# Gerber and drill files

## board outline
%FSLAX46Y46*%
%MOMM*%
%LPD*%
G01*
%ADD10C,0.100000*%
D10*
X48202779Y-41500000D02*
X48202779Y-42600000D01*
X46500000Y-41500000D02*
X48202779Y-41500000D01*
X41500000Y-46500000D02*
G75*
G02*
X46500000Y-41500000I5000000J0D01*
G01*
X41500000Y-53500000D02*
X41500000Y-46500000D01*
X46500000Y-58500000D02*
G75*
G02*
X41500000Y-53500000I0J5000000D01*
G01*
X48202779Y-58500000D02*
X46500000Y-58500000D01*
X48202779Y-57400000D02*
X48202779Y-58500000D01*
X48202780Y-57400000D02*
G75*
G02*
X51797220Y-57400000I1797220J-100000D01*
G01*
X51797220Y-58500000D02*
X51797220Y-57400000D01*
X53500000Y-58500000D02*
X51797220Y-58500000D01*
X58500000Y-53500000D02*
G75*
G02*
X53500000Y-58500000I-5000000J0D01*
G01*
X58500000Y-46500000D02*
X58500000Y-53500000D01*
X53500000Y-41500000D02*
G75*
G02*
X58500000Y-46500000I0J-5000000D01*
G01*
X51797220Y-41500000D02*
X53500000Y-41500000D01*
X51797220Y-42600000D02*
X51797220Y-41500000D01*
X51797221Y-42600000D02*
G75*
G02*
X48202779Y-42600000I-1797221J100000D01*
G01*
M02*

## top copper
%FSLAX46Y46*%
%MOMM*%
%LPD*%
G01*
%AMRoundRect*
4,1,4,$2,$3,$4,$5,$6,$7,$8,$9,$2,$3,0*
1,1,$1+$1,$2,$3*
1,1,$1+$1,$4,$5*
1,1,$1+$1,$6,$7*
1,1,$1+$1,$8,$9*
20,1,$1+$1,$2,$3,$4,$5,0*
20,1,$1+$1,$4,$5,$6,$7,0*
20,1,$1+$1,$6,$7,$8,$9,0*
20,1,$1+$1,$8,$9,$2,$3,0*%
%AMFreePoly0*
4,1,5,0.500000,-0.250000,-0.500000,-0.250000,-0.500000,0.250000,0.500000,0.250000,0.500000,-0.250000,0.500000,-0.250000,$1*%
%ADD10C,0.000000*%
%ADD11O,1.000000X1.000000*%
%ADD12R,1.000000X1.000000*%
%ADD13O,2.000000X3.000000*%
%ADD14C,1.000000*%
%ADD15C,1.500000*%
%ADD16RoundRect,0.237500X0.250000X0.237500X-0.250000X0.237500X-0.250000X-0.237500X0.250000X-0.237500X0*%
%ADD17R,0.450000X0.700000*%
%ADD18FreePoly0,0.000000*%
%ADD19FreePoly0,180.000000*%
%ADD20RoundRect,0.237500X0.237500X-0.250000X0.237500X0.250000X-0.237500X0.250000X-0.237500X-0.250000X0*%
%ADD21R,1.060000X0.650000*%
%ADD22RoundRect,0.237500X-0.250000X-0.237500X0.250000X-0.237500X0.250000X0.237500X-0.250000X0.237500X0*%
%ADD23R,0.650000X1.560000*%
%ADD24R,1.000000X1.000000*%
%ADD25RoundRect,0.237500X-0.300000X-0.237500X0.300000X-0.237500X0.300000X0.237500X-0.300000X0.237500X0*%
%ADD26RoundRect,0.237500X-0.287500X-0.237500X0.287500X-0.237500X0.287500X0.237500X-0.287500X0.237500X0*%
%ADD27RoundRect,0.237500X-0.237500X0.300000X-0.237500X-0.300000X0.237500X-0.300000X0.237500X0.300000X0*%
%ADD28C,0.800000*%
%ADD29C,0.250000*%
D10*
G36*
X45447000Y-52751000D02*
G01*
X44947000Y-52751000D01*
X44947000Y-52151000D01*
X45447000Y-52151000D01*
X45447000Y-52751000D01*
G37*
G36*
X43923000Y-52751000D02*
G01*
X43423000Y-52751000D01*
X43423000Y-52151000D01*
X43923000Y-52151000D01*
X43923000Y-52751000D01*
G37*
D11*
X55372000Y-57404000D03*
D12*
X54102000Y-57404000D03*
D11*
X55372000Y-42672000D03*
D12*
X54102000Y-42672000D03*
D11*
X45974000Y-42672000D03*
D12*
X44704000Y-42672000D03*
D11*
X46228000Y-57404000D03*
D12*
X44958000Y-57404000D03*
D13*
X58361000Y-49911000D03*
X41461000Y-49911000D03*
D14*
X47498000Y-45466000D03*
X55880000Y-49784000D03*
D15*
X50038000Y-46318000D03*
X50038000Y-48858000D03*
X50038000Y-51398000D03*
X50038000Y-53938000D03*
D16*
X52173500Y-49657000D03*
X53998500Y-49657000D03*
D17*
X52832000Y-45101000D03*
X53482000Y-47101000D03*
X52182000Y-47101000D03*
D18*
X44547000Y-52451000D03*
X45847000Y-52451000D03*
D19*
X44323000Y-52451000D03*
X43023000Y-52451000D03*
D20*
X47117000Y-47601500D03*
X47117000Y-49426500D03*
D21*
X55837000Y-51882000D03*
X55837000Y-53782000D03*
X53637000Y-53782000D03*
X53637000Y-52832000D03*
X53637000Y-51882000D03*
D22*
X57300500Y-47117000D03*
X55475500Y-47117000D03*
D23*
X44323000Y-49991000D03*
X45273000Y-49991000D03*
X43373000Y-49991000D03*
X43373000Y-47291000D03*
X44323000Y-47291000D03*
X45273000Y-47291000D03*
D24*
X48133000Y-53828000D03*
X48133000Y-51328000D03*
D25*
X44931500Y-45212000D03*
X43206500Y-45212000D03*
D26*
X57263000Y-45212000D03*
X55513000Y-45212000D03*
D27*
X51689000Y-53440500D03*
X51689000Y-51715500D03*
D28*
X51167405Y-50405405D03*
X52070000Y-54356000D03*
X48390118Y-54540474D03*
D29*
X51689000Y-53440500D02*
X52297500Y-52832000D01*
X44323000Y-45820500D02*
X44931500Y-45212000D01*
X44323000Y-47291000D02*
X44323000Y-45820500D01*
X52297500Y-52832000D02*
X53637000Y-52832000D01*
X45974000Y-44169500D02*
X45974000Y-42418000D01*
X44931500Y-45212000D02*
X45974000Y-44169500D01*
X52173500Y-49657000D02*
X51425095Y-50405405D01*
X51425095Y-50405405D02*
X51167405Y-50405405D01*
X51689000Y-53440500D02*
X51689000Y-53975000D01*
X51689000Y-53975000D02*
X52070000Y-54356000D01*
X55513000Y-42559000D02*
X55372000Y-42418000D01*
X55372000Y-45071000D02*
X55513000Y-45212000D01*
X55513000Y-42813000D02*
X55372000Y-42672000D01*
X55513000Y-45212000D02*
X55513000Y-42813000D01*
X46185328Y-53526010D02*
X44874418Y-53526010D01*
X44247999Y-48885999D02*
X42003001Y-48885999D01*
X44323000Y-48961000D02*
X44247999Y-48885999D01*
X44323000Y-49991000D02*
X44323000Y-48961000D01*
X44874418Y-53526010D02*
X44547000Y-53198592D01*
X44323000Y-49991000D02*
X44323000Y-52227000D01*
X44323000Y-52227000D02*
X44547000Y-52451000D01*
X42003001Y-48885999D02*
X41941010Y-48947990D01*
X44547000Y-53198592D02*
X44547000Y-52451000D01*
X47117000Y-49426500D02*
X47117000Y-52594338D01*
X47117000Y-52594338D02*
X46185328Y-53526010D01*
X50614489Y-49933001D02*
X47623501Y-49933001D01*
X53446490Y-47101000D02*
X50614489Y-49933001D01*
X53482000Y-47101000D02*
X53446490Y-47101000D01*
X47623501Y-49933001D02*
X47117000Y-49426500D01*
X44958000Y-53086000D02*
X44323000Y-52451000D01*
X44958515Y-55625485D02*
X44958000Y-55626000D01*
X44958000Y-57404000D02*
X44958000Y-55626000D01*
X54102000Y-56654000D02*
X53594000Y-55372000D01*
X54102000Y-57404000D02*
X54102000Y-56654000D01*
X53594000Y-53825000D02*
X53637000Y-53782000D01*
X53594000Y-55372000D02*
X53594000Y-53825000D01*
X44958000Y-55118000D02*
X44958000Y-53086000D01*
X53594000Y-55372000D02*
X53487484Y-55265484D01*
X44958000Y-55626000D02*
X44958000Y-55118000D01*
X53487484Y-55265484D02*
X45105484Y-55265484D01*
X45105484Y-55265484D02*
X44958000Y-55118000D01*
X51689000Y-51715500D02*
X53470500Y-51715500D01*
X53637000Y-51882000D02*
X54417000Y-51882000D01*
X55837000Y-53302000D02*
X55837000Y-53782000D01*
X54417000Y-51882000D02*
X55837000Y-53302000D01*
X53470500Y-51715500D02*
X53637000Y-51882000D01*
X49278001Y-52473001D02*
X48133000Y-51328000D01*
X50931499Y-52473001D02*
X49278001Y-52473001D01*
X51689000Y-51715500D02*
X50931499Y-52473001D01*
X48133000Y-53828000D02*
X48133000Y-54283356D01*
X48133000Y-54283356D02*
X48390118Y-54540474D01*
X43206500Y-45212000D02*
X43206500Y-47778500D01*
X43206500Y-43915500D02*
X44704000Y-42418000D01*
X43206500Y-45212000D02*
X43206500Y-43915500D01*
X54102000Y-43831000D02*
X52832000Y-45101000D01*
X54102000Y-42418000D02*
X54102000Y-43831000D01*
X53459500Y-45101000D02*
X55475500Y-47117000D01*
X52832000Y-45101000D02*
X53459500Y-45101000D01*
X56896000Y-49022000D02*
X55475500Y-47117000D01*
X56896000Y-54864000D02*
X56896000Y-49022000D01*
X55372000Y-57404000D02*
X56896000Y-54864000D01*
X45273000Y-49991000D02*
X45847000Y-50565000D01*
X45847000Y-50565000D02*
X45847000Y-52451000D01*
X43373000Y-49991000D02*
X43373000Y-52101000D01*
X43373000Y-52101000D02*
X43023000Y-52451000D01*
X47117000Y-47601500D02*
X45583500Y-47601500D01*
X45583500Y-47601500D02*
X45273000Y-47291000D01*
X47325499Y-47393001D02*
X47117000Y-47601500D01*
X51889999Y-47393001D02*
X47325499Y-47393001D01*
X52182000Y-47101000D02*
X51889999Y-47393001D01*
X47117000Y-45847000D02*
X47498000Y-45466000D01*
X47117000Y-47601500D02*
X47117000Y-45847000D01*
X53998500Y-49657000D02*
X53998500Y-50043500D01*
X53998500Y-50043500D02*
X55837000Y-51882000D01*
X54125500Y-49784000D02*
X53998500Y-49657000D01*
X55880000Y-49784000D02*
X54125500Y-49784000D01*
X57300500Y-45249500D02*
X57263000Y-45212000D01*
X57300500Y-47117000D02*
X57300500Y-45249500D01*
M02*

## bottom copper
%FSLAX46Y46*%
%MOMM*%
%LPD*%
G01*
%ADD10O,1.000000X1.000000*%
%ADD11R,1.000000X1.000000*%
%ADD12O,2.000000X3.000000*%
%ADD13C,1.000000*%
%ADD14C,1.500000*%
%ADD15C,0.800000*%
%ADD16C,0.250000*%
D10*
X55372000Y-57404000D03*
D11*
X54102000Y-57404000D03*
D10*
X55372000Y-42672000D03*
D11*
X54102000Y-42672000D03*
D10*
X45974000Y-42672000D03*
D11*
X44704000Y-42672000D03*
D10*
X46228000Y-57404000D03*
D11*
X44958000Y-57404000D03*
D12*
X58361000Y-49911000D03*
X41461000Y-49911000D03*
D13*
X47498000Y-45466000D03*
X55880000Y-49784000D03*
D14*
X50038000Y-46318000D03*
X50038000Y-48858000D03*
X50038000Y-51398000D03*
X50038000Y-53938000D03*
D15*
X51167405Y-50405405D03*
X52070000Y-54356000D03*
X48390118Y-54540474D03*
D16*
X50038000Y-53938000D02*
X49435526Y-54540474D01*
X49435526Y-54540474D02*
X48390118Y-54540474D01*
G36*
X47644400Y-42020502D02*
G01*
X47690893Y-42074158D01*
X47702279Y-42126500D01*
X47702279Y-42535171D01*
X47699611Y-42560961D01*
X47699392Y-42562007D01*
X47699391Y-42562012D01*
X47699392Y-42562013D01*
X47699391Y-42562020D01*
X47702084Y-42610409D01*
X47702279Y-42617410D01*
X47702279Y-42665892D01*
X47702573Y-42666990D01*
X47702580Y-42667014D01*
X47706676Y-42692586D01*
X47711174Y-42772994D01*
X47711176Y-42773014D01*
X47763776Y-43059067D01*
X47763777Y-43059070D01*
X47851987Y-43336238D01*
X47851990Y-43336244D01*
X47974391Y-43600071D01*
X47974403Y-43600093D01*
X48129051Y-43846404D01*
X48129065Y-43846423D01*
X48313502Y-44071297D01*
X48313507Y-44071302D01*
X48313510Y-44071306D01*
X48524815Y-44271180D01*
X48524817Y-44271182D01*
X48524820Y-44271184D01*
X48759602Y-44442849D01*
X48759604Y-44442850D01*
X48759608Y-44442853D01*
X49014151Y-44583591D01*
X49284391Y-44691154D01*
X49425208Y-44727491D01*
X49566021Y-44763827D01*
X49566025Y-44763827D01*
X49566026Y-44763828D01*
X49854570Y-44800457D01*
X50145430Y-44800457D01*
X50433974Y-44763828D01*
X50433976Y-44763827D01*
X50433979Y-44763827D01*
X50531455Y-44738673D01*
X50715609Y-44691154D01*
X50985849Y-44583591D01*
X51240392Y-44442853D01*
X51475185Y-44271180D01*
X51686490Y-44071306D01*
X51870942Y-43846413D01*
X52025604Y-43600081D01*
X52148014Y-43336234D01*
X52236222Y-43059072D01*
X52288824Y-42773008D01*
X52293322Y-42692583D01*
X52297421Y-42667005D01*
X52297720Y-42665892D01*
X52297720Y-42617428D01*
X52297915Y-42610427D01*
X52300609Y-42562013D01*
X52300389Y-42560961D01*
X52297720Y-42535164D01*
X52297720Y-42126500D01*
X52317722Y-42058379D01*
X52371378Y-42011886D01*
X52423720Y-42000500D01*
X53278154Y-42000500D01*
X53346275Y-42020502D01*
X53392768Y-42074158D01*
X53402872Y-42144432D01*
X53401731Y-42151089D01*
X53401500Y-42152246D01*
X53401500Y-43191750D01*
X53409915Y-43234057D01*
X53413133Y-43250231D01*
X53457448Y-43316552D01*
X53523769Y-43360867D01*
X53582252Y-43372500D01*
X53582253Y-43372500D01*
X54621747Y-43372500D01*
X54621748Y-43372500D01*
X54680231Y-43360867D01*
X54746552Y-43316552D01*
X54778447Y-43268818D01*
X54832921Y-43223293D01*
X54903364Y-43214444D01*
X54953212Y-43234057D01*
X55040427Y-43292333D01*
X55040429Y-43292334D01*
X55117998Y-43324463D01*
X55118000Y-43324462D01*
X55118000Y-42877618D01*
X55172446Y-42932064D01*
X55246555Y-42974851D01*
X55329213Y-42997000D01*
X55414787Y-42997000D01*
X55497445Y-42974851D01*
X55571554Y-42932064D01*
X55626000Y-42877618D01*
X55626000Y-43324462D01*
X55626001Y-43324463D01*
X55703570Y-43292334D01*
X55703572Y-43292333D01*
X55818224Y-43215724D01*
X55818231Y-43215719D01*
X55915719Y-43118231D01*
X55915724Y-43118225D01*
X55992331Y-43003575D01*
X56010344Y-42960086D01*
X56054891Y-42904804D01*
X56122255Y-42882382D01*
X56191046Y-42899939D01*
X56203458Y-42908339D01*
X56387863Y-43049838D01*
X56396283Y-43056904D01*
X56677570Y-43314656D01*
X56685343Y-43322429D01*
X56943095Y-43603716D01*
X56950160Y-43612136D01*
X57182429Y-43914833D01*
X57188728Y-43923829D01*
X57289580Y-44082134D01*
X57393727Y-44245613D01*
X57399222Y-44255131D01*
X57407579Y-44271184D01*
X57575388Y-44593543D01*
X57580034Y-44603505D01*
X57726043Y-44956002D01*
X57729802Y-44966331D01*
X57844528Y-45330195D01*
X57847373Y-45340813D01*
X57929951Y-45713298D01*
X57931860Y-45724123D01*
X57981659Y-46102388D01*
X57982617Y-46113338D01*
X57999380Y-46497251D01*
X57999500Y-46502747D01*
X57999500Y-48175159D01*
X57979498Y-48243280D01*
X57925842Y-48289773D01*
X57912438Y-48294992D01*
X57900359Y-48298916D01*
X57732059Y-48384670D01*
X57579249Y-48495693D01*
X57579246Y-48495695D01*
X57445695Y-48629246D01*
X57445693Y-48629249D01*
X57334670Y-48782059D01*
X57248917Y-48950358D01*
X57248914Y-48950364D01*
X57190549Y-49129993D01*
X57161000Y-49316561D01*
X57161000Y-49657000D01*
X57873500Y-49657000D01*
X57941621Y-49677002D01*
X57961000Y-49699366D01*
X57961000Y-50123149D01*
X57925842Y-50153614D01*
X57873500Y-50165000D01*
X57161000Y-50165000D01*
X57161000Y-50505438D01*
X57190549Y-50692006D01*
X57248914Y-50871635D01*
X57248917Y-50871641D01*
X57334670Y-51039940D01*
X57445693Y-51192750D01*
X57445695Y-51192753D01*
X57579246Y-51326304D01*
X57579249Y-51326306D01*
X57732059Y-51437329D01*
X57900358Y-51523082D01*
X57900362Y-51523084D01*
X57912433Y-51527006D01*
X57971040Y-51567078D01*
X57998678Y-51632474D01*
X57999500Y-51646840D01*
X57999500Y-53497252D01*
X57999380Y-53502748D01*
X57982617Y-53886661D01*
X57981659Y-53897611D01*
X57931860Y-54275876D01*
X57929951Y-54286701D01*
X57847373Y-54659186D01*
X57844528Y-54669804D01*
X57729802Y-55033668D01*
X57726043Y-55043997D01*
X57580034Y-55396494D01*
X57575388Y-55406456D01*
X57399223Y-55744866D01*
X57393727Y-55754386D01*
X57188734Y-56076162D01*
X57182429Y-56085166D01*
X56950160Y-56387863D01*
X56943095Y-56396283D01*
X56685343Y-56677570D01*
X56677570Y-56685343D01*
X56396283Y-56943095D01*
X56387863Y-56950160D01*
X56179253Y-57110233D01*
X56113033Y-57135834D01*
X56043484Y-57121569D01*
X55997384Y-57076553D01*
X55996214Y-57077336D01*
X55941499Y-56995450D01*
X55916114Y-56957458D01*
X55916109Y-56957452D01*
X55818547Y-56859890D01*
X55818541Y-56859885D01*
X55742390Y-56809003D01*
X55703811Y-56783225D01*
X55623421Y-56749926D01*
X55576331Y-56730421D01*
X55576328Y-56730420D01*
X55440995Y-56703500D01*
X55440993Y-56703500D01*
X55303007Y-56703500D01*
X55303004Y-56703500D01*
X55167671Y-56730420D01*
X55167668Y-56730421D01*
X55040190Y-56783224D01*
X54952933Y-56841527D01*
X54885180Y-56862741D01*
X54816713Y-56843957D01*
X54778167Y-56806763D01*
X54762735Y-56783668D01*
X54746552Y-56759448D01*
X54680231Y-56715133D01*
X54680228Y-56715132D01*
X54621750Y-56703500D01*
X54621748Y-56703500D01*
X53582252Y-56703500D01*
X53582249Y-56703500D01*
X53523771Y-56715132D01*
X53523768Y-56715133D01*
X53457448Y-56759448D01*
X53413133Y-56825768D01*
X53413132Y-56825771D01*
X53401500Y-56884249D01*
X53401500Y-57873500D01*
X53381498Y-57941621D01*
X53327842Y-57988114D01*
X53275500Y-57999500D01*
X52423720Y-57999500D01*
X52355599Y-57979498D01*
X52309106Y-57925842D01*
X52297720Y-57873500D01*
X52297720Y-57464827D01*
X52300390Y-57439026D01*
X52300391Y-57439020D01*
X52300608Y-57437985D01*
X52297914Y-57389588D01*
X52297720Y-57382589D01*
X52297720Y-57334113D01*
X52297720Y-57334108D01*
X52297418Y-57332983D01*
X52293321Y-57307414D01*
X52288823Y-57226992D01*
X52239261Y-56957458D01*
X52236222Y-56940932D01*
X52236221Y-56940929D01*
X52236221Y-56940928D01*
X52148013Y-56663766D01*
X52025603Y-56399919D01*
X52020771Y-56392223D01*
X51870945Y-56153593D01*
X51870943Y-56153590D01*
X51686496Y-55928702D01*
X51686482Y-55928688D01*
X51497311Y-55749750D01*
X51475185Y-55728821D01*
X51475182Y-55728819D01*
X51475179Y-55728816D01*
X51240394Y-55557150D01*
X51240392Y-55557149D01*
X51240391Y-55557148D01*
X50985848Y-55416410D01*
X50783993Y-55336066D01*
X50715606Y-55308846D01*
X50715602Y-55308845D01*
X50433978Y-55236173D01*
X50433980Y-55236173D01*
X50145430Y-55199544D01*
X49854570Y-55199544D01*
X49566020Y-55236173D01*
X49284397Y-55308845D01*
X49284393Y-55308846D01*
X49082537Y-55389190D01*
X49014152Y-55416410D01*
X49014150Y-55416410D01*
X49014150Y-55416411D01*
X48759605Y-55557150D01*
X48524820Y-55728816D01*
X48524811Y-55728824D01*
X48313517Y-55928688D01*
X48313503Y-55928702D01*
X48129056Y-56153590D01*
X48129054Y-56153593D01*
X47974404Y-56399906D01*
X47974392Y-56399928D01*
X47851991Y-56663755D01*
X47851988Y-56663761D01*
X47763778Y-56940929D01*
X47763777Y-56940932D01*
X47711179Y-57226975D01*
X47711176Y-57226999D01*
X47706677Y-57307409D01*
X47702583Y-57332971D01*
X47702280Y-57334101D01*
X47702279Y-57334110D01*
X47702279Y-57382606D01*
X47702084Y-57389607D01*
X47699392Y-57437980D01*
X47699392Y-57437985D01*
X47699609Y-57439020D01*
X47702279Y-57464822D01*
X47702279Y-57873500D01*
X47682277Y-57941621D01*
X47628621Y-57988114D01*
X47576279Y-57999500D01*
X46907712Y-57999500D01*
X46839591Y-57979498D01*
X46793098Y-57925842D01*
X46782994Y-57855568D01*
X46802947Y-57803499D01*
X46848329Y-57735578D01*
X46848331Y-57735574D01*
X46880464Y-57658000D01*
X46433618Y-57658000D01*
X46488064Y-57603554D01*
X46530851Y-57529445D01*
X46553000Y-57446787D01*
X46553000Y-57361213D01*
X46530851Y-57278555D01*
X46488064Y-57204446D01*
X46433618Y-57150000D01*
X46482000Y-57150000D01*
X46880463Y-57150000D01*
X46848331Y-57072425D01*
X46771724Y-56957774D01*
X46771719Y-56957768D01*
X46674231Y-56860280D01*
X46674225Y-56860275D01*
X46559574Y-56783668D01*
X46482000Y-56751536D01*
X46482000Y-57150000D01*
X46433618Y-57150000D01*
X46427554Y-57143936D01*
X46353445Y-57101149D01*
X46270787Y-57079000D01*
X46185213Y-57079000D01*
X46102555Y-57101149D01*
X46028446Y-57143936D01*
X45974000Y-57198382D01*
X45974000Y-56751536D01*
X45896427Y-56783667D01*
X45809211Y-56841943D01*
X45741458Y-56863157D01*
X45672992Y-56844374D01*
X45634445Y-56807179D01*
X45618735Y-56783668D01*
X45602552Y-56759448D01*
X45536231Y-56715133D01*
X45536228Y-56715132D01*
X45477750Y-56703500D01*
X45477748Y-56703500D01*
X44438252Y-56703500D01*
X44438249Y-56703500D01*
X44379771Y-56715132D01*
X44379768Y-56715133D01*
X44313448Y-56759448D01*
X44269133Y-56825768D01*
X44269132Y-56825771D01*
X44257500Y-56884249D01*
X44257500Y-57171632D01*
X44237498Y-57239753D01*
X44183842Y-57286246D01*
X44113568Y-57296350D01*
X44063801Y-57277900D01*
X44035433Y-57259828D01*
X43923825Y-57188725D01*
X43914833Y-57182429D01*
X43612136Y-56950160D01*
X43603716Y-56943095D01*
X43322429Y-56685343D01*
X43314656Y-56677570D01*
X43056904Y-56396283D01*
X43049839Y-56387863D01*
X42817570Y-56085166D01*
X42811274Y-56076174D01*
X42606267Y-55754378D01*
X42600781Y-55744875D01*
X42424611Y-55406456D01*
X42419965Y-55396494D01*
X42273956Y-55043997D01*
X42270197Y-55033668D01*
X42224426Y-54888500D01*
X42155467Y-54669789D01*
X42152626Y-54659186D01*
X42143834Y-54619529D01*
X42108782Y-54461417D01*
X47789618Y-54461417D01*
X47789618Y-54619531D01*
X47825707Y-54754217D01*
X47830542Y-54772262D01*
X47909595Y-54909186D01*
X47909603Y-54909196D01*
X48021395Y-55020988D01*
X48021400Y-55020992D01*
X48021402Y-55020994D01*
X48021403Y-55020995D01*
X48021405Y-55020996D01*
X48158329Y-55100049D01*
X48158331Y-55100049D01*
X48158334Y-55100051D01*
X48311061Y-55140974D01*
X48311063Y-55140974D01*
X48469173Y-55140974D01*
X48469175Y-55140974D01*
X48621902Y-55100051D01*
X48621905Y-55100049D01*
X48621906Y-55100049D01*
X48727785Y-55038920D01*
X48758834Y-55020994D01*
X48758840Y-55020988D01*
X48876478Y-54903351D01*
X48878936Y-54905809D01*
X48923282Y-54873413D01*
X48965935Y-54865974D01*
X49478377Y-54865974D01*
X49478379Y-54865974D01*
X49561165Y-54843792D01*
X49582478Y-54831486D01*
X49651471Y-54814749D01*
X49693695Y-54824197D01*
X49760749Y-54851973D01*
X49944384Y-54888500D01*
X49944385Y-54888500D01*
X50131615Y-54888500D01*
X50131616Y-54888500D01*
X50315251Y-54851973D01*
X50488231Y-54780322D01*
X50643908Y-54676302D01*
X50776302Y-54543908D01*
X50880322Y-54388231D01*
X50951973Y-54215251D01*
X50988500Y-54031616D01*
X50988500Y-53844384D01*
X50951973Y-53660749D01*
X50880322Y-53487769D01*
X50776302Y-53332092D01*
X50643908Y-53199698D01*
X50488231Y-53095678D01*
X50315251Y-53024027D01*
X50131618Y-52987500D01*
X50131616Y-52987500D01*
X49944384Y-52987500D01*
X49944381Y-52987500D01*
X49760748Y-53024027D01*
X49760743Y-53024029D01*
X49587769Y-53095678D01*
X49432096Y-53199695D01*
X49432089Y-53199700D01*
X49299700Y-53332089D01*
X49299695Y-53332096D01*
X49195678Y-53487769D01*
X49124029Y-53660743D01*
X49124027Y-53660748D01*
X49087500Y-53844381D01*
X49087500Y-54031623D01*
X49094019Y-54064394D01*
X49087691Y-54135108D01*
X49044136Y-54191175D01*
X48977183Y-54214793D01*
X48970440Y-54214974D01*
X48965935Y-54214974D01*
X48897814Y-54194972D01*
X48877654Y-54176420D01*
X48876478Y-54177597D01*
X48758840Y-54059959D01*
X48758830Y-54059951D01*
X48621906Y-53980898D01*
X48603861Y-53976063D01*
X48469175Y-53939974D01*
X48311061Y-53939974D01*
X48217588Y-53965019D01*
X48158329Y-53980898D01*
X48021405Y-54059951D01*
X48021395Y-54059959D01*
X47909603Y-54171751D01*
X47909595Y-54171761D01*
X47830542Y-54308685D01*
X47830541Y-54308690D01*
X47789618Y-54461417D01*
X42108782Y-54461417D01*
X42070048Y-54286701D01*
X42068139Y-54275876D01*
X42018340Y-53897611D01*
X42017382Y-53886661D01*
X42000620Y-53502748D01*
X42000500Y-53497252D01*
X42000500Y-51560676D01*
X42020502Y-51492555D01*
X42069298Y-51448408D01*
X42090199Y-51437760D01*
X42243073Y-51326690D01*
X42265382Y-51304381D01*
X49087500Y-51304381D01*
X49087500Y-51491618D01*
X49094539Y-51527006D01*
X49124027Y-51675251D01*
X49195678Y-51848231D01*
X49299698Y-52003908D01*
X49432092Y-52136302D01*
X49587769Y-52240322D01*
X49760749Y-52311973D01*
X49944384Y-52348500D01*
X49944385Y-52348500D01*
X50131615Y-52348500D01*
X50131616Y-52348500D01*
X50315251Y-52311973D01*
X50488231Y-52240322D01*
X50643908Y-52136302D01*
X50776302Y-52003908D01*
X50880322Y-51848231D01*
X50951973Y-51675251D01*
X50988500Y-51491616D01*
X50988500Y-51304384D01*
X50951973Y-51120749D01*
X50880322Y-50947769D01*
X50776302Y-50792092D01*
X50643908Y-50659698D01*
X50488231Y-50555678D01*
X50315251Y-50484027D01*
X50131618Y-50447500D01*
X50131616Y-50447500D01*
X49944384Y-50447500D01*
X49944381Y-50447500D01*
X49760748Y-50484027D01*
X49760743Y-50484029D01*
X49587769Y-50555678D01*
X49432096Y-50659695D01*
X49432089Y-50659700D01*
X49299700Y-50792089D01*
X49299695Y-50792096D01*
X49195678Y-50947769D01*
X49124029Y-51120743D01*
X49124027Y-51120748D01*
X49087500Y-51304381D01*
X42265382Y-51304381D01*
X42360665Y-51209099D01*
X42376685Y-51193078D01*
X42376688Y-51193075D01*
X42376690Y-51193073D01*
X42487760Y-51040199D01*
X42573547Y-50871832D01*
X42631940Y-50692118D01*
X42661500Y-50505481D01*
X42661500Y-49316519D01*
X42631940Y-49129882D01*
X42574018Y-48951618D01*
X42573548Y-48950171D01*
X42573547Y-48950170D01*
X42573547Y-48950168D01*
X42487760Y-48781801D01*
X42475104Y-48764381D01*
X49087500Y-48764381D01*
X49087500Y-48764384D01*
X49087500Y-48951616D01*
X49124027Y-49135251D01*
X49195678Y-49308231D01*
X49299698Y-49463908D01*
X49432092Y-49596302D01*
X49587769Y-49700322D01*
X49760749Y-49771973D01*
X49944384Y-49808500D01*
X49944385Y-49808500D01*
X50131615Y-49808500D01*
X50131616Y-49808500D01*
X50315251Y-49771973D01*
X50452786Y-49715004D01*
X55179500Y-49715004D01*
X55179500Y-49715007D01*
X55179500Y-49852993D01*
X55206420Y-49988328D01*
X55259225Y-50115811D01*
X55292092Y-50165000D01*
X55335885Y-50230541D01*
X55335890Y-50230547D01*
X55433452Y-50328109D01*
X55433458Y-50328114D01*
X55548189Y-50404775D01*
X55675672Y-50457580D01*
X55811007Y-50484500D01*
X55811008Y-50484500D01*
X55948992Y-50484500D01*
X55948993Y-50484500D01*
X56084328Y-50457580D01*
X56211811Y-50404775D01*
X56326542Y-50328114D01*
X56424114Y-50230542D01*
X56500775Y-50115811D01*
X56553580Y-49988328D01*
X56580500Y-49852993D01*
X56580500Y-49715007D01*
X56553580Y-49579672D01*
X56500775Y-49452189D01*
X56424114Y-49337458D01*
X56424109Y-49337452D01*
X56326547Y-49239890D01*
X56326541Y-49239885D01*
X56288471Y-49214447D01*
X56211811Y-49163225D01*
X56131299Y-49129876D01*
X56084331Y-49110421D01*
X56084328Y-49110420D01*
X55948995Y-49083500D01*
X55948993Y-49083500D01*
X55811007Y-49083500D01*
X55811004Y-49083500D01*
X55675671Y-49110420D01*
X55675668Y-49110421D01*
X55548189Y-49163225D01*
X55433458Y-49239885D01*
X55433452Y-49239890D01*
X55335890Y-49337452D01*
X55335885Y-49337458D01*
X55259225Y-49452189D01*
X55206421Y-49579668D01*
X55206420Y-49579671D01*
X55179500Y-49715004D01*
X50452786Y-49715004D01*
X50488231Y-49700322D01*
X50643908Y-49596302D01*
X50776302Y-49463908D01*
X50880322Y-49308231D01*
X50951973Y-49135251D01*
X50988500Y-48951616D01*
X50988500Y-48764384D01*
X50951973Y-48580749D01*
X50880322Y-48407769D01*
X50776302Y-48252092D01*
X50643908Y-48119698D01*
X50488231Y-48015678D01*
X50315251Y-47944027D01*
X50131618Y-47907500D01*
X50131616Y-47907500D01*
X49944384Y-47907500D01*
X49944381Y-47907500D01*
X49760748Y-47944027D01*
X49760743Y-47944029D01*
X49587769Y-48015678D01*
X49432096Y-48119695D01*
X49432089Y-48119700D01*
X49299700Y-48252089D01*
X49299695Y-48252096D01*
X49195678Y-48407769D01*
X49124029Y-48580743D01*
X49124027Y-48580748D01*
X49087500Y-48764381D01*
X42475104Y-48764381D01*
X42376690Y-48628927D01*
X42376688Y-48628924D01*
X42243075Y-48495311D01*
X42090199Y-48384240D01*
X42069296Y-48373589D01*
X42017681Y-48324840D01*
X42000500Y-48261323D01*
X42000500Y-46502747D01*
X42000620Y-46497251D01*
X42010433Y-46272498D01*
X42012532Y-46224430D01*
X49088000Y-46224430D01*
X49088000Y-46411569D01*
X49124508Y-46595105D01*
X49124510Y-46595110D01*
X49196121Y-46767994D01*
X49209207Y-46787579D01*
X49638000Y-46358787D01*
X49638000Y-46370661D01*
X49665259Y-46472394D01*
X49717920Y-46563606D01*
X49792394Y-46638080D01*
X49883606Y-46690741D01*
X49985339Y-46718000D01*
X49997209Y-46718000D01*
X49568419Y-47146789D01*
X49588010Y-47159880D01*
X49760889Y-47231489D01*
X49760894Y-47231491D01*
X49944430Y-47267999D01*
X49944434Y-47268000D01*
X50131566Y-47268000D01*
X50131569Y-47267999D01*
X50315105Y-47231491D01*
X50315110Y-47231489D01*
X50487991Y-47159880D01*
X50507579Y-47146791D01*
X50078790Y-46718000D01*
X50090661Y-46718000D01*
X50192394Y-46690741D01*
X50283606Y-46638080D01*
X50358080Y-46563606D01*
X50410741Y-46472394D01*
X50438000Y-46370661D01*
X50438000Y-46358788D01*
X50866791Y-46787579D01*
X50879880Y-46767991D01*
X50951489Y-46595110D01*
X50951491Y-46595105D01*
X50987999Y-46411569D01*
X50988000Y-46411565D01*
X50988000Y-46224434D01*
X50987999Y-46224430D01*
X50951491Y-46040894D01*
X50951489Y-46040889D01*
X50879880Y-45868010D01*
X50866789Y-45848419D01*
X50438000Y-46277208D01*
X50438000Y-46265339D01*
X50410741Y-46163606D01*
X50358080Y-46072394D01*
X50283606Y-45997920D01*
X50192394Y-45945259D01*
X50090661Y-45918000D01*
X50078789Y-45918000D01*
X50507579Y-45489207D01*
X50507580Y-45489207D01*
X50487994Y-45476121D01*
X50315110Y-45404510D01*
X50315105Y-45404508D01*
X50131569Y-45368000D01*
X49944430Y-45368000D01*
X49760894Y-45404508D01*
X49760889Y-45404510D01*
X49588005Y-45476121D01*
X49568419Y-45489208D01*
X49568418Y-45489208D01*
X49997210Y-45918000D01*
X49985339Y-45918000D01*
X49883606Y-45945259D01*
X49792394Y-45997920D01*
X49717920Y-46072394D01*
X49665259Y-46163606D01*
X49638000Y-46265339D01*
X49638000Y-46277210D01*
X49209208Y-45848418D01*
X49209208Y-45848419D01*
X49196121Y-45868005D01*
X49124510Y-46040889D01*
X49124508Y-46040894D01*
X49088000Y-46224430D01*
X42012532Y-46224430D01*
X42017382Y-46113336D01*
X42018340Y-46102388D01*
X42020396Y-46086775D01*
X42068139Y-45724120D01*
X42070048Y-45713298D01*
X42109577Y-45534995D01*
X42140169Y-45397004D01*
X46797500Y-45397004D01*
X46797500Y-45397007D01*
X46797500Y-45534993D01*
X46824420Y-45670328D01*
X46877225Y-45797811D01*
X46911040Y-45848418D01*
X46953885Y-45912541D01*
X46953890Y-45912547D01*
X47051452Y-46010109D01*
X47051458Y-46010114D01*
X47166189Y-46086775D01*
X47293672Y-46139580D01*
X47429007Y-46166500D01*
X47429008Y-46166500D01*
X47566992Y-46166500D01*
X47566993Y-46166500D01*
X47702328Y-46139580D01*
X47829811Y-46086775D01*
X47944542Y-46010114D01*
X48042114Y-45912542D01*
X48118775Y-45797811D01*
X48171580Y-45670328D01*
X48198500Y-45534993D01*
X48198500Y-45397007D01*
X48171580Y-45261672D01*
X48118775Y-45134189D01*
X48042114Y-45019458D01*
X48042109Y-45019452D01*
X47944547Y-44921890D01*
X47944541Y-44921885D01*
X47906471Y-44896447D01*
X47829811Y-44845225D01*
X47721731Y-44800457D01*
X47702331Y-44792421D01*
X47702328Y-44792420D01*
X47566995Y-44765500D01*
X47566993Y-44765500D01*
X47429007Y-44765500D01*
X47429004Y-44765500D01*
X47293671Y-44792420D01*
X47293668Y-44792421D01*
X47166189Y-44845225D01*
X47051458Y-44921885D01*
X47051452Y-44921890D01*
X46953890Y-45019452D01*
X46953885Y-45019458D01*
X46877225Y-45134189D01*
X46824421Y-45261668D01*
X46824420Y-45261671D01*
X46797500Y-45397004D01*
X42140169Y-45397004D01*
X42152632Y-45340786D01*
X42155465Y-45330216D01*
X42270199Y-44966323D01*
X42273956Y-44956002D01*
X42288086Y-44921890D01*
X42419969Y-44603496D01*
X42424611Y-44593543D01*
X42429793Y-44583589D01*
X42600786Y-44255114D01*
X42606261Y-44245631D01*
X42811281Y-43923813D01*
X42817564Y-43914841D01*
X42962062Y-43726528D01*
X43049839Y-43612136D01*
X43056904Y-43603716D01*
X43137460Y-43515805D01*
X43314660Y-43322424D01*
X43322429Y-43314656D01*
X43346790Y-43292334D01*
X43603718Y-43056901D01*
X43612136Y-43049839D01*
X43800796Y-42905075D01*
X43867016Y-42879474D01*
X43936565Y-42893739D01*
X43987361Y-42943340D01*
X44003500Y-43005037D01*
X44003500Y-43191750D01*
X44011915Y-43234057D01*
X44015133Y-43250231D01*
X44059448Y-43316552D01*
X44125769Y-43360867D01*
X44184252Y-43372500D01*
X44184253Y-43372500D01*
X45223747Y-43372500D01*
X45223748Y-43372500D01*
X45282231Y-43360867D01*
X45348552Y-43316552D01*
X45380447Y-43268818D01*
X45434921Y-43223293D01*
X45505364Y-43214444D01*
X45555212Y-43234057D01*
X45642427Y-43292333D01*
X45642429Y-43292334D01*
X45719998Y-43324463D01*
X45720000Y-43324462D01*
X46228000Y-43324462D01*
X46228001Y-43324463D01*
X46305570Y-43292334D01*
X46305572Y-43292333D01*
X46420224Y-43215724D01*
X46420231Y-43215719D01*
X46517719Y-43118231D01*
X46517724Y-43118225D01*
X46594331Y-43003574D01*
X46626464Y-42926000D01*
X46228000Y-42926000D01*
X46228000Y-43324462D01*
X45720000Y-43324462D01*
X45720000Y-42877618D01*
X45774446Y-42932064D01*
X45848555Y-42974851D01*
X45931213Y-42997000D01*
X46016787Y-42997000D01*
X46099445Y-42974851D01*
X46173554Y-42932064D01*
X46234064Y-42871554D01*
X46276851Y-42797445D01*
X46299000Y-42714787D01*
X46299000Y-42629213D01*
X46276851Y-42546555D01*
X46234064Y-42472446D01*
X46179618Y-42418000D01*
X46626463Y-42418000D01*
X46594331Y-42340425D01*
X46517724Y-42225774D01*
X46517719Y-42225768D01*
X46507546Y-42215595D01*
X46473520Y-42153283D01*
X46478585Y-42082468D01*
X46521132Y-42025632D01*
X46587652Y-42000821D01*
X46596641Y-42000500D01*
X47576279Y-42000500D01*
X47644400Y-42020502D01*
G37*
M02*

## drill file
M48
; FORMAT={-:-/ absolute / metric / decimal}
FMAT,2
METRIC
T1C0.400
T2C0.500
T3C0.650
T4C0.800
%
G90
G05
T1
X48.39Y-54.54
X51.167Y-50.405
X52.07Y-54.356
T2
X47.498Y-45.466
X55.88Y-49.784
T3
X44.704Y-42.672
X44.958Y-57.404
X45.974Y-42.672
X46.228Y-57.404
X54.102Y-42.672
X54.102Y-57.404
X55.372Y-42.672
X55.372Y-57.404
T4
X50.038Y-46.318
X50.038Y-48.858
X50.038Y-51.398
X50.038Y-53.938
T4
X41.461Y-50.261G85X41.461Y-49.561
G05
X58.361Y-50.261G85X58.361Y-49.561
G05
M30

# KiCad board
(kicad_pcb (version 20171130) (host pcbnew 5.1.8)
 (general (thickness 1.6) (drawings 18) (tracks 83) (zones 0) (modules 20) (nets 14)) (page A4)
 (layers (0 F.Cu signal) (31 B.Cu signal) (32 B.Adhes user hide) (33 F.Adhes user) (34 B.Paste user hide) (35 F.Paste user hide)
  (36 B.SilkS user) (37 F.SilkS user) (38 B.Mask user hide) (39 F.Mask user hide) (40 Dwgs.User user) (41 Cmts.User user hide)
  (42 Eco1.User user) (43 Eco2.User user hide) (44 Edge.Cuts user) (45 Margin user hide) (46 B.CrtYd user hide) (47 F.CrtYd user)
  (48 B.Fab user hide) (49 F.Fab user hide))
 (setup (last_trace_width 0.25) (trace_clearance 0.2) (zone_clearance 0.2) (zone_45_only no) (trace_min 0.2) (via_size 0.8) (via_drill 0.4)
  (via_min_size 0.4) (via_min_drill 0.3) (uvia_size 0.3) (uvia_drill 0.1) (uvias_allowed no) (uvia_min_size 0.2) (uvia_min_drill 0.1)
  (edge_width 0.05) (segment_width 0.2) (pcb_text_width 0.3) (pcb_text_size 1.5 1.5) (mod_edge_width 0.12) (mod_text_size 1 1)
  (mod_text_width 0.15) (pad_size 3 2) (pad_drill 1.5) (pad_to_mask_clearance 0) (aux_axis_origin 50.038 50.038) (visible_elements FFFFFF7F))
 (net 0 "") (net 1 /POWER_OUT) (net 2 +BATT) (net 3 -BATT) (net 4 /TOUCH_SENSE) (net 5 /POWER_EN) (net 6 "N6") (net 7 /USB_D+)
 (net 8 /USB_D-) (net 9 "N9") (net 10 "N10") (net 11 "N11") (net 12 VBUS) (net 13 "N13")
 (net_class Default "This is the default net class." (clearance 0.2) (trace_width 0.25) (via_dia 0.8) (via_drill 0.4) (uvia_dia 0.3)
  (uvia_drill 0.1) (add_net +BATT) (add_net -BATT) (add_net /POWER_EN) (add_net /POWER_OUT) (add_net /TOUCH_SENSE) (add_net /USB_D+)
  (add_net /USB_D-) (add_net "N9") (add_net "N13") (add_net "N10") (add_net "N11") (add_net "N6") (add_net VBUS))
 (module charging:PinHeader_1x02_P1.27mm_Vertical (layer F.Cu) (at 54.102 57.404 90)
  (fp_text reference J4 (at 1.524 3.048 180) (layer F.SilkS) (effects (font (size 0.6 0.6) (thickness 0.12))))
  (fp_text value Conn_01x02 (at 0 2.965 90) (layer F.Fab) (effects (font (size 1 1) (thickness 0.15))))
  (pad 2 thru_hole oval (at 0 1.27 90) (size 1 1) (drill 0.65) (layers *.Cu *.Mask) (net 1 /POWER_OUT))
  (pad 1 thru_hole rect (at 0 0 90) (size 1 1) (drill 0.65) (layers *.Cu *.Mask) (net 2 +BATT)))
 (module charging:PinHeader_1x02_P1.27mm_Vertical (layer F.Cu) (at 54.102 42.672 90)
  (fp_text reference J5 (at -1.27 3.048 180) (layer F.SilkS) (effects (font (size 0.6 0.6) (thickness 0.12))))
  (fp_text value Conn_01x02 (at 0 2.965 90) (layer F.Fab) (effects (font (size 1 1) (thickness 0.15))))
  (pad 2 thru_hole oval (at 0 1.27 90) (size 1 1) (drill 0.65) (layers *.Cu *.Mask) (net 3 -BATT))
  (pad 1 thru_hole rect (at 0 0 90) (size 1 1) (drill 0.65) (layers *.Cu *.Mask) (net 1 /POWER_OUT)))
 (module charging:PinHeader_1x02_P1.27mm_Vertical (layer F.Cu) (at 44.704 42.672 90)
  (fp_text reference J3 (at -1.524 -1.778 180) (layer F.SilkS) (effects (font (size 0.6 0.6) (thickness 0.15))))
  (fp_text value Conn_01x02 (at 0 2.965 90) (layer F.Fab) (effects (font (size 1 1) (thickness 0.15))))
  (pad 2 thru_hole oval (at 0 1.27 90) (size 1 1) (drill 0.65) (layers *.Cu *.Mask) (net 3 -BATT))
  (pad 1 thru_hole rect (at 0 0 90) (size 1 1) (drill 0.65) (layers *.Cu *.Mask) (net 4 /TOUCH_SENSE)))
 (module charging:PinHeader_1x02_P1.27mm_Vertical (layer F.Cu) (at 44.958 57.404 90)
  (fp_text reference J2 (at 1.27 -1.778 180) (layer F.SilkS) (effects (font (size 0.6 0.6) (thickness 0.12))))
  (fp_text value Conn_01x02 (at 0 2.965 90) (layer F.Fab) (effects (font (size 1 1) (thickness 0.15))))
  (pad 2 thru_hole oval (at 0 1.27 90) (size 1 1) (drill 0.65) (layers *.Cu *.Mask) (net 3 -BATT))
  (pad 1 thru_hole rect (at 0 0 90) (size 1 1) (drill 0.65) (layers *.Cu *.Mask) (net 2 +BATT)))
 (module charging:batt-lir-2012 (layer F.Cu) (at 49.911 49.911 90)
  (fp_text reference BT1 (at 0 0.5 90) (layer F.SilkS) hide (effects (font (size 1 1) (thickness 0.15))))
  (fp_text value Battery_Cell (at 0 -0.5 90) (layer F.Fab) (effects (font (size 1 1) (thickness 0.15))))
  (pad 2 thru_hole oval (at 0 8.45 90) (size 3 2) (drill oval 1.5 0.8) (layers *.Cu *.Mask) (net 3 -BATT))
  (pad 1 thru_hole oval (at 0 -8.45 90) (size 3 2) (drill oval 1.5 0.8) (layers *.Cu *.Mask) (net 2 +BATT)))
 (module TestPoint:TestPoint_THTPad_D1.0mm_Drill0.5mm (layer F.Cu) (at 47.498 45.466)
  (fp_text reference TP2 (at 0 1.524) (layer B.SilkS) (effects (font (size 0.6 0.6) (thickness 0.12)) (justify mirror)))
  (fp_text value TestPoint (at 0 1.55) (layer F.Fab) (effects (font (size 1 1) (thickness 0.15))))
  (pad 1 thru_hole circle (at 0 0) (size 1 1) (drill 0.5) (layers *.Cu *.Mask) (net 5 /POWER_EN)))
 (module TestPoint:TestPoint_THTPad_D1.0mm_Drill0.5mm (layer F.Cu) (at 55.88 49.784)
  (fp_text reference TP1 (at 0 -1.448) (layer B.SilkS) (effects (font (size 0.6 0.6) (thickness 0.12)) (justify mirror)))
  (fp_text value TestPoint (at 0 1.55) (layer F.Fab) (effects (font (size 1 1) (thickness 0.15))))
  (pad 1 thru_hole circle (at 0 0) (size 1 1) (drill 0.5) (layers *.Cu *.Mask) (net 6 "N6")))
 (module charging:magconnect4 (layer F.Cu) (at 50.038 50.038)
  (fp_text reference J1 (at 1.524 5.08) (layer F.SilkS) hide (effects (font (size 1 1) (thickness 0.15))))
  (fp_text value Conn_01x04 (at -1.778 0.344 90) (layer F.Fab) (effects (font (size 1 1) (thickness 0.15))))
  (pad 4 thru_hole circle (at 0 -3.72) (size 1.5 1.5) (drill 0.8) (layers B.Cu B.Mask) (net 3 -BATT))
  (pad 3 thru_hole circle (at 0 -1.18) (size 1.5 1.5) (drill 0.8) (layers B.Cu B.Mask) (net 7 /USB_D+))
  (pad 2 thru_hole circle (at 0 1.36) (size 1.5 1.5) (drill 0.8) (layers B.Cu B.Mask) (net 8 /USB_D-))
  (pad 1 thru_hole circle (at 0 3.9) (size 1.5 1.5) (drill 0.8) (layers B.Cu B.Mask) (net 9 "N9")))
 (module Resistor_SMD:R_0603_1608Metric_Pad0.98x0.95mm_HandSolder (layer F.Cu) (at 53.086 49.657 180)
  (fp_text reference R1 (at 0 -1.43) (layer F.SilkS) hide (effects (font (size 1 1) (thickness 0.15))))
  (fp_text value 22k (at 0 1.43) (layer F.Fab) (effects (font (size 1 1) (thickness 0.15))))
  (pad 2 smd roundrect (at 0.9125 0 180) (size 0.975 0.95) (layers F.Cu F.Paste F.Mask) (roundrect_rratio 0.25) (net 3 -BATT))
  (pad 1 smd roundrect (at -0.9125 0 180) (size 0.975 0.95) (layers F.Cu F.Paste F.Mask) (roundrect_rratio 0.25) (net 6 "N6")))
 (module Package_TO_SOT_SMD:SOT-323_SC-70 (layer F.Cu) (at 52.832 46.101 90)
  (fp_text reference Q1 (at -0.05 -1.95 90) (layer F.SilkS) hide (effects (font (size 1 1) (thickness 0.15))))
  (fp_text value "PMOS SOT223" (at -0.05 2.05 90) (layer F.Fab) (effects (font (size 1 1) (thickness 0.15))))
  (pad 3 smd rect (at 1 0) (size 0.45 0.7) (layers F.Cu F.Paste F.Mask) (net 1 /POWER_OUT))
  (pad 2 smd rect (at -1 0.65) (size 0.45 0.7) (layers F.Cu F.Paste F.Mask) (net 2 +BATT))
  (pad 1 smd rect (at -1 -0.65) (size 0.45 0.7) (layers F.Cu F.Paste F.Mask) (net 5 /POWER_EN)))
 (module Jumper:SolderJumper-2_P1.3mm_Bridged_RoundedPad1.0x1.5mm (layer F.Cu) (at 45.197 52.451)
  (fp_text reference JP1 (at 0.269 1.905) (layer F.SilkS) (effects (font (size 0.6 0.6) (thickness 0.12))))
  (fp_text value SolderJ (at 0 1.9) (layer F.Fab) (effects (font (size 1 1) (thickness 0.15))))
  (fp_poly (pts (xy 0.25 -0.3) (xy -0.25 -0.3) (xy -0.25 0.3) (xy 0.25 0.3)) (layer F.Cu) (width 0))
  (pad 1 smd custom (at -0.65 0) (size 1 0.5) (layers F.Cu F.Mask) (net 2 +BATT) (zone_connect 2)
   (options (clearance outline) (anchor rect)) (primitives))
  (pad 2 smd custom (at 0.65 0) (size 1 0.5) (layers F.Cu F.Mask) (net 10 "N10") (zone_connect 2)
   (options (clearance outline) (anchor rect)) (primitives)))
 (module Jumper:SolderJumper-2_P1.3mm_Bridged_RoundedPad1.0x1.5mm (layer F.Cu) (at 43.673 52.451 180)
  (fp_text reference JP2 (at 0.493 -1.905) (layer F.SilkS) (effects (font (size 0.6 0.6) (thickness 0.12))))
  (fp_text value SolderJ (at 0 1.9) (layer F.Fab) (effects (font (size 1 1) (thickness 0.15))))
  (fp_poly (pts (xy 0.25 -0.3) (xy -0.25 -0.3) (xy -0.25 0.3) (xy 0.25 0.3)) (layer F.Cu) (width 0))
  (pad 1 smd custom (at -0.65 0 180) (size 1 0.5) (layers F.Cu F.Mask) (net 2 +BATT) (zone_connect 2)
   (options (clearance outline) (anchor rect)) (primitives))
  (pad 2 smd custom (at 0.65 0 180) (size 1 0.5) (layers F.Cu F.Mask) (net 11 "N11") (zone_connect 2)
   (options (clearance outline) (anchor rect)) (primitives)))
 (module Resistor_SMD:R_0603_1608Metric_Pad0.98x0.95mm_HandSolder (layer F.Cu) (at 47.117 48.514 90)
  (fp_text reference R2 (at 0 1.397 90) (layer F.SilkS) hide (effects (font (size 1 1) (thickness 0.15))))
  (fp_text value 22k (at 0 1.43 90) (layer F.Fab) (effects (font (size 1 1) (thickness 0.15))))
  (pad 2 smd roundrect (at 0.9125 0 90) (size 0.975 0.95) (layers F.Cu F.Paste F.Mask) (roundrect_rratio 0.25) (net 5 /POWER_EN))
  (pad 1 smd roundrect (at -0.9125 0 90) (size 0.975 0.95) (layers F.Cu F.Paste F.Mask) (roundrect_rratio 0.25) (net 2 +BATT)))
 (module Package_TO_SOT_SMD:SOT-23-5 (layer F.Cu) (at 54.737 52.832)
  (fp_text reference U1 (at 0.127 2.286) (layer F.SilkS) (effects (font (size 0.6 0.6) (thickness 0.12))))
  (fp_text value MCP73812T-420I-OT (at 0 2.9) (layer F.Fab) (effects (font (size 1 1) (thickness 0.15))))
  (pad 5 smd rect (at 1.1 -0.95) (size 1.06 0.65) (layers F.Cu F.Paste F.Mask) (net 6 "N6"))
  (pad 4 smd rect (at 1.1 0.95) (size 1.06 0.65) (layers F.Cu F.Paste F.Mask) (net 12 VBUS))
  (pad 3 smd rect (at -1.1 0.95) (size 1.06 0.65) (layers F.Cu F.Paste F.Mask) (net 2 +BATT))
  (pad 2 smd rect (at -1.1 0) (size 1.06 0.65) (layers F.Cu F.Paste F.Mask) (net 3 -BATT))
  (pad 1 smd rect (at -1.1 -0.95) (size 1.06 0.65) (layers F.Cu F.Paste F.Mask) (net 12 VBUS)))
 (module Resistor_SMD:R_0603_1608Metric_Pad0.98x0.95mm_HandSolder (layer F.Cu) (at 56.388 47.117)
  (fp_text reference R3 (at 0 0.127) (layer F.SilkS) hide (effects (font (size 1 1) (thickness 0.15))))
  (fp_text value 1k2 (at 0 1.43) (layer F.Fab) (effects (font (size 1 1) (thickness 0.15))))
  (pad 2 smd roundrect (at 0.9125 0) (size 0.975 0.95) (layers F.Cu F.Paste F.Mask) (roundrect_rratio 0.25) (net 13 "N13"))
  (pad 1 smd roundrect (at -0.9125 0) (size 0.975 0.95) (layers F.Cu F.Paste F.Mask) (roundrect_rratio 0.25) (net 1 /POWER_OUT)))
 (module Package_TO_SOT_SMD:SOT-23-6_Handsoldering (layer F.Cu) (at 44.323 48.641 270)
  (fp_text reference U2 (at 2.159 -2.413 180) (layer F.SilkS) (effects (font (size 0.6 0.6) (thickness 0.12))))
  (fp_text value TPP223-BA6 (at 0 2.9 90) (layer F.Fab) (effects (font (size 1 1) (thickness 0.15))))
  (pad 5 smd rect (at 1.35 0 270) (size 1.56 0.65) (layers F.Cu F.Paste F.Mask) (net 2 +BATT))
  (pad 6 smd rect (at 1.35 -0.95 270) (size 1.56 0.65) (layers F.Cu F.Paste F.Mask) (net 10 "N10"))
  (pad 4 smd rect (at 1.35 0.95 270) (size 1.56 0.65) (layers F.Cu F.Paste F.Mask) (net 11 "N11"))
  (pad 3 smd rect (at -1.35 0.95 270) (size 1.56 0.65) (layers F.Cu F.Paste F.Mask) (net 4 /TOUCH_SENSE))
  (pad 2 smd rect (at -1.35 0 270) (size 1.56 0.65) (layers F.Cu F.Paste F.Mask) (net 3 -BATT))
  (pad 1 smd rect (at -1.35 -0.95 270) (size 1.56 0.65) (layers F.Cu F.Paste F.Mask) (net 5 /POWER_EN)))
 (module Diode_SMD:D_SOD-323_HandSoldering (layer F.Cu) (at 48.133 52.578 270)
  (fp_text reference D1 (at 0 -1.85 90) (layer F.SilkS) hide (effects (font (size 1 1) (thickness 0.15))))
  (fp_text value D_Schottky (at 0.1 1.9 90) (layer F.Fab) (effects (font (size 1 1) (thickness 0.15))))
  (pad 2 smd rect (at 1.25 0 270) (size 1 1) (layers F.Cu F.Paste F.Mask) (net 9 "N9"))
  (pad 1 smd rect (at -1.25 0 270) (size 1 1) (layers F.Cu F.Paste F.Mask) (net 12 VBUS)))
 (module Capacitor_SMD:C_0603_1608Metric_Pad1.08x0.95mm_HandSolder (layer F.Cu) (at 44.069 45.212)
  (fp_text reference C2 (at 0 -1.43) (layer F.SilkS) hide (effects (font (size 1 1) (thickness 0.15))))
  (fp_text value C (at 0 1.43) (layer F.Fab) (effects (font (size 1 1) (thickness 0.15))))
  (pad 2 smd roundrect (at 0.8625 0) (size 1.075 0.95) (layers F.Cu F.Paste F.Mask) (roundrect_rratio 0.25) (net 3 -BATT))
  (pad 1 smd roundrect (at -0.8625 0) (size 1.075 0.95) (layers F.Cu F.Paste F.Mask) (roundrect_rratio 0.25) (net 4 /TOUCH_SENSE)))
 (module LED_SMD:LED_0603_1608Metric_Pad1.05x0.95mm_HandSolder (layer F.Cu) (at 56.388 45.212)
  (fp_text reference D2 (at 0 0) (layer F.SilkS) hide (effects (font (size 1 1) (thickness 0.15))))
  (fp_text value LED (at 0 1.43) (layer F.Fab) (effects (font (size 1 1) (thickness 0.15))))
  (pad 2 smd roundrect (at 0.875 0) (size 1.05 0.95) (layers F.Cu F.Paste F.Mask) (roundrect_rratio 0.25) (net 13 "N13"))
  (pad 1 smd roundrect (at -0.875 0) (size 1.05 0.95) (layers F.Cu F.Paste F.Mask) (roundrect_rratio 0.25) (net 3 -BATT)))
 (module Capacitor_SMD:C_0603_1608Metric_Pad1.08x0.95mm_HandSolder (layer F.Cu) (at 51.689 52.578 270)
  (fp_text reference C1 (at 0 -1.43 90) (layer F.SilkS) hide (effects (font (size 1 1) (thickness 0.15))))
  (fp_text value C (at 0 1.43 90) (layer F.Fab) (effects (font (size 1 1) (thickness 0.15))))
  (pad 2 smd roundrect (at 0.8625 0 270) (size 1.075 0.95) (layers F.Cu F.Paste F.Mask) (roundrect_rratio 0.25) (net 3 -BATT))
  (pad 1 smd roundrect (at -0.8625 0 270) (size 1.075 0.95) (layers F.Cu F.Paste F.Mask) (roundrect_rratio 0.25) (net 12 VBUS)))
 (gr_line (start 48.202779 41.5) (end 48.202779 42.6) (layer Edge.Cuts) (width 0.1))
 (gr_line (start 46.5 41.5) (end 48.202779 41.5) (layer Edge.Cuts) (width 0.1))
 (gr_arc (start 46.5 46.5) (end 46.5 41.5) (angle -90) (layer Edge.Cuts) (width 0.1))
 (gr_line (start 41.5 53.5) (end 41.5 46.5) (layer Edge.Cuts) (width 0.1))
 (gr_arc (start 46.5 53.5) (end 41.5 53.5) (angle -90) (layer Edge.Cuts) (width 0.1))
 (gr_line (start 48.202779 58.5) (end 46.5 58.5) (layer Edge.Cuts) (width 0.1))
 (gr_line (start 48.202779 57.4) (end 48.202779 58.5) (layer Edge.Cuts) (width 0.1))
 (gr_arc (start 50 57.5) (end 51.79722 57.4) (angle -173.6305229) (layer Edge.Cuts) (width 0.1))
 (gr_line (start 51.79722 58.5) (end 51.79722 57.4) (layer Edge.Cuts) (width 0.1))
 (gr_line (start 53.5 58.5) (end 51.79722 58.5) (layer Edge.Cuts) (width 0.1))
 (gr_arc (start 53.5 53.5) (end 53.5 58.5) (angle -90) (layer Edge.Cuts) (width 0.1))
 (gr_line (start 58.5 46.5) (end 58.5 53.5) (layer Edge.Cuts) (width 0.1))
 (gr_arc (start 53.5 46.5) (end 58.5 46.5) (angle -90) (layer Edge.Cuts) (width 0.1))
 (gr_line (start 51.79722 41.5) (end 53.5 41.5) (layer Edge.Cuts) (width 0.1))
 (gr_line (start 51.79722 42.6) (end 51.79722 41.5) (layer Edge.Cuts) (width 0.1))
 (gr_arc (start 50 42.5) (end 48.202779 42.6) (angle -173.6305229) (layer Edge.Cuts) (width 0.1))
 (segment (start 51.689 53.4405) (end 52.2975 52.832) (width 0.25) (layer F.Cu) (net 3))
 (segment (start 44.323 45.8205) (end 44.9315 45.212) (width 0.25) (layer F.Cu) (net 3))
 (segment (start 44.323 47.291) (end 44.323 45.8205) (width 0.25) (layer F.Cu) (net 3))
 (segment (start 52.2975 52.832) (end 53.637 52.832) (width 0.25) (layer F.Cu) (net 3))
 (segment (start 45.974 44.1695) (end 45.974 42.418) (width 0.25) (layer F.Cu) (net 3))
 (segment (start 44.9315 45.212) (end 45.974 44.1695) (width 0.25) (layer F.Cu) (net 3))
 (via (at 51.167405 50.405405) (size 0.8) (drill 0.4) (layers F.Cu B.Cu) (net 3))
 (segment (start 52.1735 49.657) (end 51.425095 50.405405) (width 0.25) (layer F.Cu) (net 3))
 (segment (start 51.425095 50.405405) (end 51.167405 50.405405) (width 0.25) (layer F.Cu) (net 3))
 (segment (start 51.689 53.4405) (end 51.689 53.975) (width 0.25) (layer F.Cu) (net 3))
 (via (at 52.07 54.356) (size 0.8) (drill 0.4) (layers F.Cu B.Cu) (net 3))
 (segment (start 51.689 53.975) (end 52.07 54.356) (width 0.25) (layer F.Cu) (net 3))
 (segment (start 55.513 42.559) (end 55.372 42.418) (width 0.25) (layer F.Cu) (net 3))
 (segment (start 55.372 45.071) (end 55.513 45.212) (width 0.25) (layer F.Cu) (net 3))
 (segment (start 55.513 42.813) (end 55.372 42.672) (width 0.25) (layer F.Cu) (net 3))
 (segment (start 55.513 45.212) (end 55.513 42.813) (width 0.25) (layer F.Cu) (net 3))
 (segment (start 46.185328 53.52601) (end 44.874418 53.52601) (width 0.25) (layer F.Cu) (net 2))
 (segment (start 44.247999 48.885999) (end 42.003001 48.885999) (width 0.25) (layer F.Cu) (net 2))
 (segment (start 44.323 48.961) (end 44.247999 48.885999) (width 0.25) (layer F.Cu) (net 2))
 (segment (start 44.323 49.991) (end 44.323 48.961) (width 0.25) (layer F.Cu) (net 2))
 (segment (start 44.874418 53.52601) (end 44.547 53.198592) (width 0.25) (layer F.Cu) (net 2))
 (segment (start 44.323 49.991) (end 44.323 52.227) (width 0.25) (layer F.Cu) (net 2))
 (segment (start 44.323 52.227) (end 44.547 52.451) (width 0.25) (layer F.Cu) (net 2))
 (segment (start 42.003001 48.885999) (end 41.94101 48.94799) (width 0.25) (layer F.Cu) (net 2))
 (segment (start 44.547 53.198592) (end 44.547 52.451) (width 0.25) (layer F.Cu) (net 2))
 (segment (start 47.117 49.4265) (end 47.117 52.594338) (width 0.25) (layer F.Cu) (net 2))
 (segment (start 47.117 52.594338) (end 46.185328 53.52601) (width 0.25) (layer F.Cu) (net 2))
 (segment (start 50.614489 49.933001) (end 47.623501 49.933001) (width 0.25) (layer F.Cu) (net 2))
 (segment (start 53.44649 47.101) (end 50.614489 49.933001) (width 0.25) (layer F.Cu) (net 2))
 (segment (start 53.482 47.101) (end 53.44649 47.101) (width 0.25) (layer F.Cu) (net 2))
 (segment (start 47.623501 49.933001) (end 47.117 49.4265) (width 0.25) (layer F.Cu) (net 2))
 (segment (start 44.958 53.086) (end 44.323 52.451) (width 0.25) (layer F.Cu) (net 2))
 (segment (start 44.958515 55.625485) (end 44.958 55.626) (width 0.25) (layer F.Cu) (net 2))
 (segment (start 44.958 57.404) (end 44.958 55.626) (width 0.25) (layer F.Cu) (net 2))
 (segment (start 54.102 56.654) (end 53.594 55.372) (width 0.25) (layer F.Cu) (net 2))
 (segment (start 54.102 57.404) (end 54.102 56.654) (width 0.25) (layer F.Cu) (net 2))
 (segment (start 53.594 53.825) (end 53.637 53.782) (width 0.25) (layer F.Cu) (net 2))
 (segment (start 53.594 55.372) (end 53.594 53.825) (width 0.25) (layer F.Cu) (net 2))
 (segment (start 44.958 55.118) (end 44.958 53.086) (width 0.25) (layer F.Cu) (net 2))
 (segment (start 53.594 55.372) (end 53.487484 55.265484) (width 0.25) (layer F.Cu) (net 2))
 (segment (start 44.958 55.626) (end 44.958 55.118) (width 0.25) (layer F.Cu) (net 2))
 (segment (start 53.487484 55.265484) (end 45.105484 55.265484) (width 0.25) (layer F.Cu) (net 2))
 (segment (start 45.105484 55.265484) (end 44.958 55.118) (width 0.25) (layer F.Cu) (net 2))
 (segment (start 51.689 51.7155) (end 53.4705 51.7155) (width 0.25) (layer F.Cu) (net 12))
 (segment (start 53.637 51.882) (end 54.417 51.882) (width 0.25) (layer F.Cu) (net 12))
 (segment (start 55.837 53.302) (end 55.837 53.782) (width 0.25) (layer F.Cu) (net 12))
 (segment (start 54.417 51.882) (end 55.837 53.302) (width 0.25) (layer F.Cu) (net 12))
 (segment (start 53.4705 51.7155) (end 53.637 51.882) (width 0.25) (layer F.Cu) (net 12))
 (segment (start 49.278001 52.473001) (end 48.133 51.328) (width 0.25) (layer F.Cu) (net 12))
 (segment (start 50.931499 52.473001) (end 49.278001 52.473001) (width 0.25) (layer F.Cu) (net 12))
 (segment (start 51.689 51.7155) (end 50.931499 52.473001) (width 0.25) (layer F.Cu) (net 12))
 (segment (start 48.133 53.828) (end 48.133 54.283356) (width 0.25) (layer F.Cu) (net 9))
 (via (at 48.390118 54.540474) (size 0.8) (drill 0.4) (layers F.Cu B.Cu) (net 9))
 (segment (start 48.133 54.283356) (end 48.390118 54.540474) (width 0.25) (layer F.Cu) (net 9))
 (segment (start 50.038 53.938) (end 49.435526 54.540474) (width 0.25) (layer B.Cu) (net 9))
 (segment (start 49.435526 54.540474) (end 48.390118 54.540474) (width 0.25) (layer B.Cu) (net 9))
 (segment (start 43.2065 45.212) (end 43.2065 47.7785) (width 0.25) (layer F.Cu) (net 4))
 (segment (start 43.2065 43.9155) (end 44.704 42.418) (width 0.25) (layer F.Cu) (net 4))
 (segment (start 43.2065 45.212) (end 43.2065 43.9155) (width 0.25) (layer F.Cu) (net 4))
 (segment (start 54.102 43.831) (end 52.832 45.101) (width 0.25) (layer F.Cu) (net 1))
 (segment (start 54.102 42.418) (end 54.102 43.831) (width 0.25) (layer F.Cu) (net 1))
 (segment (start 53.4595 45.101) (end 55.4755 47.117) (width 0.25) (layer F.Cu) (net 1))
 (segment (start 52.832 45.101) (end 53.4595 45.101) (width 0.25) (layer F.Cu) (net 1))
 (segment (start 56.896 49.022) (end 55.4755 47.117) (width 0.25) (layer F.Cu) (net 1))
 (segment (start 56.896 54.864) (end 56.896 49.022) (width 0.25) (layer F.Cu) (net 1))
 (segment (start 55.372 57.404) (end 56.896 54.864) (width 0.25) (layer F.Cu) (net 1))
 (segment (start 45.273 49.991) (end 45.847 50.565) (width 0.25) (layer F.Cu) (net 10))
 (segment (start 45.847 50.565) (end 45.847 52.451) (width 0.25) (layer F.Cu) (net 10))
 (segment (start 43.373 49.991) (end 43.373 52.101) (width 0.25) (layer F.Cu) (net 11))
 (segment (start 43.373 52.101) (end 43.023 52.451) (width 0.25) (layer F.Cu) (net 11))
 (segment (start 47.117 47.6015) (end 45.5835 47.6015) (width 0.25) (layer F.Cu) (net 5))
 (segment (start 45.5835 47.6015) (end 45.273 47.291) (width 0.25) (layer F.Cu) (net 5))
 (segment (start 47.325499 47.393001) (end 47.117 47.6015) (width 0.25) (layer F.Cu) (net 5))
 (segment (start 51.889999 47.393001) (end 47.325499 47.393001) (width 0.25) (layer F.Cu) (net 5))
 (segment (start 52.182 47.101) (end 51.889999 47.393001) (width 0.25) (layer F.Cu) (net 5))
 (segment (start 47.117 45.847) (end 47.498 45.466) (width 0.25) (layer F.Cu) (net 5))
 (segment (start 47.117 47.6015) (end 47.117 45.847) (width 0.25) (layer F.Cu) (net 5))
 (segment (start 53.9985 49.657) (end 53.9985 50.0435) (width 0.25) (layer F.Cu) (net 6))
 (segment (start 53.9985 50.0435) (end 55.837 51.882) (width 0.25) (layer F.Cu) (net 6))
 (segment (start 54.1255 49.784) (end 53.9985 49.657) (width 0.25) (layer F.Cu) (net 6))
 (segment (start 55.88 49.784) (end 54.1255 49.784) (width 0.25) (layer F.Cu) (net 6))
 (segment (start 57.3005 45.2495) (end 57.263 45.212) (width 0.25) (layer F.Cu) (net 13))
 (segment (start 57.3005 47.117) (end 57.3005 45.2495) (width 0.25) (layer F.Cu) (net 13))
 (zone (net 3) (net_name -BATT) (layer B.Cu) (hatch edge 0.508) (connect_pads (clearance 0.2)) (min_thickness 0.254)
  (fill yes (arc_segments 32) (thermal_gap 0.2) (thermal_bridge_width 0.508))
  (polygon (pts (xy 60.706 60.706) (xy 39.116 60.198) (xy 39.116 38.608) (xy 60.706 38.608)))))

